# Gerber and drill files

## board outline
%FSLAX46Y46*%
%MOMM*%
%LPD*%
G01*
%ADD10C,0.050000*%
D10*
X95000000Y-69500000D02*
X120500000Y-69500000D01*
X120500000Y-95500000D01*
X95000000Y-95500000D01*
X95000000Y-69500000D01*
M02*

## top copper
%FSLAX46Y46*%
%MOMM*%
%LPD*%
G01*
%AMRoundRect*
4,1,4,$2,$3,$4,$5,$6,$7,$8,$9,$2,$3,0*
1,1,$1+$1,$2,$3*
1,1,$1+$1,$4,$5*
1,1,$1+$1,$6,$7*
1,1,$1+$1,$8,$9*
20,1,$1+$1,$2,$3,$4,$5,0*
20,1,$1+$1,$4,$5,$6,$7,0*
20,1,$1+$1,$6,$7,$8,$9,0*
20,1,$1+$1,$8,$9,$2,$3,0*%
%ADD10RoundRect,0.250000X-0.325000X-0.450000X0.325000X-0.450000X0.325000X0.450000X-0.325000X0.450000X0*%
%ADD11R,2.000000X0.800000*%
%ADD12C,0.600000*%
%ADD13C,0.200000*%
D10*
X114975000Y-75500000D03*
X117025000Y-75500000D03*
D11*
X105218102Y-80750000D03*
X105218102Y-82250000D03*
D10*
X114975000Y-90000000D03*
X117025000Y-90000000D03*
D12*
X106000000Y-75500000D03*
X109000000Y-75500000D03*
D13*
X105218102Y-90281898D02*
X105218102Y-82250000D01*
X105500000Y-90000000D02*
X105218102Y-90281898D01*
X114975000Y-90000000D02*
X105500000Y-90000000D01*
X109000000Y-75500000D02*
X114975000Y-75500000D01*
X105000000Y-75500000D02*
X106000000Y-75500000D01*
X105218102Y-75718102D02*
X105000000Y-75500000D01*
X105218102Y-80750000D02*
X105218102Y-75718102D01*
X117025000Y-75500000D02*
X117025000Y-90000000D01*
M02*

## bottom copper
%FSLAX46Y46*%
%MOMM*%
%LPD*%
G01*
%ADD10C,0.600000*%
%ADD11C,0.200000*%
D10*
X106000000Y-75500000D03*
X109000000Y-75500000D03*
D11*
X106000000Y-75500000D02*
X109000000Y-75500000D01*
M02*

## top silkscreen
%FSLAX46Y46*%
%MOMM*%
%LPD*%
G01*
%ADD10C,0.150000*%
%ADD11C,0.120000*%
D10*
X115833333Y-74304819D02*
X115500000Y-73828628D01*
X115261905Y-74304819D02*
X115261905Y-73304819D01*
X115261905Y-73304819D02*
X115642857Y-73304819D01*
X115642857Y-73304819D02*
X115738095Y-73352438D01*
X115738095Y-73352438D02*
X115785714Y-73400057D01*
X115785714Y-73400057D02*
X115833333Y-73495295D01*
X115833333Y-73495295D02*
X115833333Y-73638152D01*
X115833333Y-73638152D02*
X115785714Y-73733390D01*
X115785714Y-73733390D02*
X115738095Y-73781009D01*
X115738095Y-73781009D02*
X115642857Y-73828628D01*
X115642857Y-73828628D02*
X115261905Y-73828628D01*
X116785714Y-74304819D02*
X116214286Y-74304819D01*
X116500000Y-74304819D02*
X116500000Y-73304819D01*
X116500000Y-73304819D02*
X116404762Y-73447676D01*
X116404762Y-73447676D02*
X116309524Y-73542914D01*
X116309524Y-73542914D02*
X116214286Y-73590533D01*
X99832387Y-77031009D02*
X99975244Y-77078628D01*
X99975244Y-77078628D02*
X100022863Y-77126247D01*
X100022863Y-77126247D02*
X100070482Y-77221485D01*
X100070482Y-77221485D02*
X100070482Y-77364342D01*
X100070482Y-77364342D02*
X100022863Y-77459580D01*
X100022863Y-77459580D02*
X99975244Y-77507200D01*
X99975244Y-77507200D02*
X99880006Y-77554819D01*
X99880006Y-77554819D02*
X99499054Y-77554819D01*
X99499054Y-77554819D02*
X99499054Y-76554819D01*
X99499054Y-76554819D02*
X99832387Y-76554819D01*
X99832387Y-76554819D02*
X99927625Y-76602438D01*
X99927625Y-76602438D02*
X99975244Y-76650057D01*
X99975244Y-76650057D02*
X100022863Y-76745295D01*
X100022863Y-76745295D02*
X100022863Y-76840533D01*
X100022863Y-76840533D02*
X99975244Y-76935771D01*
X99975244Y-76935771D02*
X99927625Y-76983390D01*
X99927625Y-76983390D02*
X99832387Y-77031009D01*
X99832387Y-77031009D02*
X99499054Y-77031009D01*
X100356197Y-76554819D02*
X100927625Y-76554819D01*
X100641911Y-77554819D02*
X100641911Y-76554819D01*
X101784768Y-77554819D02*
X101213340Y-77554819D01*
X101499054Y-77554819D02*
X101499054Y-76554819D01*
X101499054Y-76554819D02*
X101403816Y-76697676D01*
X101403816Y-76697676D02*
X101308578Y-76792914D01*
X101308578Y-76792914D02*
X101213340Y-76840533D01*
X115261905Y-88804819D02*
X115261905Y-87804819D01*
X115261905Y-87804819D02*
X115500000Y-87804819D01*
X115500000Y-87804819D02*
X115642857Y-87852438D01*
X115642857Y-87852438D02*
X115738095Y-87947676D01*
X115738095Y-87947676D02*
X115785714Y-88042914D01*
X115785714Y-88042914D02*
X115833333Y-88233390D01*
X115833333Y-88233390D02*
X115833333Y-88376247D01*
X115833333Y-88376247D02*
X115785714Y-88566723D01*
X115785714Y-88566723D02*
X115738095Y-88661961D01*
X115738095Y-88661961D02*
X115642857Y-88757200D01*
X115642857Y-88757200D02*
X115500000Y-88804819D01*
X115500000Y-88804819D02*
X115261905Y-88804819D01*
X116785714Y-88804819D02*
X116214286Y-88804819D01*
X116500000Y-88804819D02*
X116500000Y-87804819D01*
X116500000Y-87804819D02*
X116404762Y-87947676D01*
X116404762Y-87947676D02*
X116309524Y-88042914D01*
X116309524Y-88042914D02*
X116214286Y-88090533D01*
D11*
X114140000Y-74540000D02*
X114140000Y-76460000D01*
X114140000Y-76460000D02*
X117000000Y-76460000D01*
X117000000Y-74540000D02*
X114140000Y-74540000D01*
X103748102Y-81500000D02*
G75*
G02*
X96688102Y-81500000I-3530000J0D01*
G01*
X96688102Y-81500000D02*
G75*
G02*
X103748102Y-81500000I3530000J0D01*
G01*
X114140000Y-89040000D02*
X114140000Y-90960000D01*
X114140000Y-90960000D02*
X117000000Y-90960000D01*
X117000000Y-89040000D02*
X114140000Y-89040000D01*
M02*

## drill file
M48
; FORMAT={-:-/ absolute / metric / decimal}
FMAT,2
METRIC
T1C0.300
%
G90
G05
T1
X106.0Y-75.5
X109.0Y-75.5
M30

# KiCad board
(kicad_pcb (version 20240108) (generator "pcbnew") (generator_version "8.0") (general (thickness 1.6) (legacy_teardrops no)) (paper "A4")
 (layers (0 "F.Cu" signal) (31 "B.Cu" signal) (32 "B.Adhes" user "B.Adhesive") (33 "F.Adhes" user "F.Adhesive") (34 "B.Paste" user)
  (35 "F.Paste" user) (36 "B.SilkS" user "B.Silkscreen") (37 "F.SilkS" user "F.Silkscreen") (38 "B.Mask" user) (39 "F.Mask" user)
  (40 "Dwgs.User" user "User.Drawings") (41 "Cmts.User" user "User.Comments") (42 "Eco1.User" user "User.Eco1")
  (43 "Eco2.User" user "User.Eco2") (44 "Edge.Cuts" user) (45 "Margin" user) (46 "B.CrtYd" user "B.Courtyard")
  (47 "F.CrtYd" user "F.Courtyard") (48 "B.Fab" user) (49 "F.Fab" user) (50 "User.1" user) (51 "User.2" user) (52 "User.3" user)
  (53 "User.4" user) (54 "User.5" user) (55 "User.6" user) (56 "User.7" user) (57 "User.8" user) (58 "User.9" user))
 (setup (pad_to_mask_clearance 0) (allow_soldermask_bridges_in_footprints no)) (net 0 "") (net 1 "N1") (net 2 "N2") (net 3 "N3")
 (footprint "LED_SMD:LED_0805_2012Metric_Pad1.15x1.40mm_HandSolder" (layer "F.Cu") (at 116 75.5)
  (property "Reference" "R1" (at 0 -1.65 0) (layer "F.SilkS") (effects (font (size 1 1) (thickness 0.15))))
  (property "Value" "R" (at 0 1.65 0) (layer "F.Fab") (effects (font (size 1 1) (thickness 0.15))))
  (fp_line (start -1.86 -0.96) (end -1.86 0.96) (stroke (width 0.12) (type solid)) (layer "F.SilkS"))
  (fp_line (start -1.86 0.96) (end 1 0.96) (stroke (width 0.12) (type solid)) (layer "F.SilkS"))
  (fp_line (start 1 -0.96) (end -1.86 -0.96) (stroke (width 0.12) (type solid)) (layer "F.SilkS"))
  (pad "1" smd roundrect (at -1.025 0) (size 1.15 1.4) (layers "F.Cu" "F.Paste" "F.Mask") (roundrect_rratio 0.217391) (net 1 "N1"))
  (pad "2" smd roundrect (at 1.025 0) (size 1.15 1.4) (layers "F.Cu" "F.Paste" "F.Mask") (roundrect_rratio 0.217391) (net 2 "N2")))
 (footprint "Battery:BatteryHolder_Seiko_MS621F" (layer "F.Cu") (at 105.218102 81.5)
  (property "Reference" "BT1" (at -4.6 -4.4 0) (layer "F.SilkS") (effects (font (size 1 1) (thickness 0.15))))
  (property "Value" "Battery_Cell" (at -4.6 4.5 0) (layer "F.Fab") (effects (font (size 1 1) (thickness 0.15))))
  (fp_circle (center -5 0) (end -1.47 0) (stroke (width 0.12) (type solid)) (fill none) (layer "F.SilkS"))
  (pad "1" smd rect (at 0 -0.75) (size 2 0.8) (layers "F.Cu" "F.Paste" "F.Mask") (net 1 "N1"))
  (pad "2" smd rect (at 0 0.75) (size 2 0.8) (layers "F.Cu" "F.Paste" "F.Mask") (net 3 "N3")))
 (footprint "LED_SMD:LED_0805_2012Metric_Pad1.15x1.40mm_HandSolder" (layer "F.Cu") (at 116 90)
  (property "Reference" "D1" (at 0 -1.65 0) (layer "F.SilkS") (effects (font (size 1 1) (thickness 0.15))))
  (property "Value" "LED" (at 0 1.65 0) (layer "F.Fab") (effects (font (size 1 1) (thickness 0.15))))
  (fp_line (start -1.86 -0.96) (end -1.86 0.96) (stroke (width 0.12) (type solid)) (layer "F.SilkS"))
  (fp_line (start -1.86 0.96) (end 1 0.96) (stroke (width 0.12) (type solid)) (layer "F.SilkS"))
  (fp_line (start 1 -0.96) (end -1.86 -0.96) (stroke (width 0.12) (type solid)) (layer "F.SilkS"))
  (pad "1" smd roundrect (at -1.025 0) (size 1.15 1.4) (layers "F.Cu" "F.Paste" "F.Mask") (roundrect_rratio 0.217391) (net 3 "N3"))
  (pad "2" smd roundrect (at 1.025 0) (size 1.15 1.4) (layers "F.Cu" "F.Paste" "F.Mask") (roundrect_rratio 0.217391) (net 2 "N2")))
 (gr_rect (start 95 69.5) (end 120.5 95.5) (stroke (width 0.05) (type default)) (fill none) (layer "Edge.Cuts"))
 (segment (start 105.218102 90.281898) (end 105.218102 82.25) (width 0.2) (layer "F.Cu") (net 3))
 (segment (start 105.5 90) (end 105.218102 90.281898) (width 0.2) (layer "F.Cu") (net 3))
 (segment (start 114.975 90) (end 105.5 90) (width 0.2) (layer "F.Cu") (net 3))
 (segment (start 109 75.5) (end 114.975 75.5) (width 0.2) (layer "F.Cu") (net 1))
 (segment (start 105 75.5) (end 106 75.5) (width 0.2) (layer "F.Cu") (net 1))
 (segment (start 105.218102 75.718102) (end 105 75.5) (width 0.2) (layer "F.Cu") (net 1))
 (segment (start 105.218102 80.75) (end 105.218102 75.718102) (width 0.2) (layer "F.Cu") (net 1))
 (via (at 106 75.5) (size 0.6) (drill 0.3) (layers "F.Cu" "B.Cu") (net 1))
 (via (at 109 75.5) (size 0.6) (drill 0.3) (layers "F.Cu" "B.Cu") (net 1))
 (segment (start 106 75.5) (end 109 75.5) (width 0.2) (layer "B.Cu") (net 1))
 (segment (start 117.025 75.5) (end 117.025 90) (width 0.2) (layer "F.Cu") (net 2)))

